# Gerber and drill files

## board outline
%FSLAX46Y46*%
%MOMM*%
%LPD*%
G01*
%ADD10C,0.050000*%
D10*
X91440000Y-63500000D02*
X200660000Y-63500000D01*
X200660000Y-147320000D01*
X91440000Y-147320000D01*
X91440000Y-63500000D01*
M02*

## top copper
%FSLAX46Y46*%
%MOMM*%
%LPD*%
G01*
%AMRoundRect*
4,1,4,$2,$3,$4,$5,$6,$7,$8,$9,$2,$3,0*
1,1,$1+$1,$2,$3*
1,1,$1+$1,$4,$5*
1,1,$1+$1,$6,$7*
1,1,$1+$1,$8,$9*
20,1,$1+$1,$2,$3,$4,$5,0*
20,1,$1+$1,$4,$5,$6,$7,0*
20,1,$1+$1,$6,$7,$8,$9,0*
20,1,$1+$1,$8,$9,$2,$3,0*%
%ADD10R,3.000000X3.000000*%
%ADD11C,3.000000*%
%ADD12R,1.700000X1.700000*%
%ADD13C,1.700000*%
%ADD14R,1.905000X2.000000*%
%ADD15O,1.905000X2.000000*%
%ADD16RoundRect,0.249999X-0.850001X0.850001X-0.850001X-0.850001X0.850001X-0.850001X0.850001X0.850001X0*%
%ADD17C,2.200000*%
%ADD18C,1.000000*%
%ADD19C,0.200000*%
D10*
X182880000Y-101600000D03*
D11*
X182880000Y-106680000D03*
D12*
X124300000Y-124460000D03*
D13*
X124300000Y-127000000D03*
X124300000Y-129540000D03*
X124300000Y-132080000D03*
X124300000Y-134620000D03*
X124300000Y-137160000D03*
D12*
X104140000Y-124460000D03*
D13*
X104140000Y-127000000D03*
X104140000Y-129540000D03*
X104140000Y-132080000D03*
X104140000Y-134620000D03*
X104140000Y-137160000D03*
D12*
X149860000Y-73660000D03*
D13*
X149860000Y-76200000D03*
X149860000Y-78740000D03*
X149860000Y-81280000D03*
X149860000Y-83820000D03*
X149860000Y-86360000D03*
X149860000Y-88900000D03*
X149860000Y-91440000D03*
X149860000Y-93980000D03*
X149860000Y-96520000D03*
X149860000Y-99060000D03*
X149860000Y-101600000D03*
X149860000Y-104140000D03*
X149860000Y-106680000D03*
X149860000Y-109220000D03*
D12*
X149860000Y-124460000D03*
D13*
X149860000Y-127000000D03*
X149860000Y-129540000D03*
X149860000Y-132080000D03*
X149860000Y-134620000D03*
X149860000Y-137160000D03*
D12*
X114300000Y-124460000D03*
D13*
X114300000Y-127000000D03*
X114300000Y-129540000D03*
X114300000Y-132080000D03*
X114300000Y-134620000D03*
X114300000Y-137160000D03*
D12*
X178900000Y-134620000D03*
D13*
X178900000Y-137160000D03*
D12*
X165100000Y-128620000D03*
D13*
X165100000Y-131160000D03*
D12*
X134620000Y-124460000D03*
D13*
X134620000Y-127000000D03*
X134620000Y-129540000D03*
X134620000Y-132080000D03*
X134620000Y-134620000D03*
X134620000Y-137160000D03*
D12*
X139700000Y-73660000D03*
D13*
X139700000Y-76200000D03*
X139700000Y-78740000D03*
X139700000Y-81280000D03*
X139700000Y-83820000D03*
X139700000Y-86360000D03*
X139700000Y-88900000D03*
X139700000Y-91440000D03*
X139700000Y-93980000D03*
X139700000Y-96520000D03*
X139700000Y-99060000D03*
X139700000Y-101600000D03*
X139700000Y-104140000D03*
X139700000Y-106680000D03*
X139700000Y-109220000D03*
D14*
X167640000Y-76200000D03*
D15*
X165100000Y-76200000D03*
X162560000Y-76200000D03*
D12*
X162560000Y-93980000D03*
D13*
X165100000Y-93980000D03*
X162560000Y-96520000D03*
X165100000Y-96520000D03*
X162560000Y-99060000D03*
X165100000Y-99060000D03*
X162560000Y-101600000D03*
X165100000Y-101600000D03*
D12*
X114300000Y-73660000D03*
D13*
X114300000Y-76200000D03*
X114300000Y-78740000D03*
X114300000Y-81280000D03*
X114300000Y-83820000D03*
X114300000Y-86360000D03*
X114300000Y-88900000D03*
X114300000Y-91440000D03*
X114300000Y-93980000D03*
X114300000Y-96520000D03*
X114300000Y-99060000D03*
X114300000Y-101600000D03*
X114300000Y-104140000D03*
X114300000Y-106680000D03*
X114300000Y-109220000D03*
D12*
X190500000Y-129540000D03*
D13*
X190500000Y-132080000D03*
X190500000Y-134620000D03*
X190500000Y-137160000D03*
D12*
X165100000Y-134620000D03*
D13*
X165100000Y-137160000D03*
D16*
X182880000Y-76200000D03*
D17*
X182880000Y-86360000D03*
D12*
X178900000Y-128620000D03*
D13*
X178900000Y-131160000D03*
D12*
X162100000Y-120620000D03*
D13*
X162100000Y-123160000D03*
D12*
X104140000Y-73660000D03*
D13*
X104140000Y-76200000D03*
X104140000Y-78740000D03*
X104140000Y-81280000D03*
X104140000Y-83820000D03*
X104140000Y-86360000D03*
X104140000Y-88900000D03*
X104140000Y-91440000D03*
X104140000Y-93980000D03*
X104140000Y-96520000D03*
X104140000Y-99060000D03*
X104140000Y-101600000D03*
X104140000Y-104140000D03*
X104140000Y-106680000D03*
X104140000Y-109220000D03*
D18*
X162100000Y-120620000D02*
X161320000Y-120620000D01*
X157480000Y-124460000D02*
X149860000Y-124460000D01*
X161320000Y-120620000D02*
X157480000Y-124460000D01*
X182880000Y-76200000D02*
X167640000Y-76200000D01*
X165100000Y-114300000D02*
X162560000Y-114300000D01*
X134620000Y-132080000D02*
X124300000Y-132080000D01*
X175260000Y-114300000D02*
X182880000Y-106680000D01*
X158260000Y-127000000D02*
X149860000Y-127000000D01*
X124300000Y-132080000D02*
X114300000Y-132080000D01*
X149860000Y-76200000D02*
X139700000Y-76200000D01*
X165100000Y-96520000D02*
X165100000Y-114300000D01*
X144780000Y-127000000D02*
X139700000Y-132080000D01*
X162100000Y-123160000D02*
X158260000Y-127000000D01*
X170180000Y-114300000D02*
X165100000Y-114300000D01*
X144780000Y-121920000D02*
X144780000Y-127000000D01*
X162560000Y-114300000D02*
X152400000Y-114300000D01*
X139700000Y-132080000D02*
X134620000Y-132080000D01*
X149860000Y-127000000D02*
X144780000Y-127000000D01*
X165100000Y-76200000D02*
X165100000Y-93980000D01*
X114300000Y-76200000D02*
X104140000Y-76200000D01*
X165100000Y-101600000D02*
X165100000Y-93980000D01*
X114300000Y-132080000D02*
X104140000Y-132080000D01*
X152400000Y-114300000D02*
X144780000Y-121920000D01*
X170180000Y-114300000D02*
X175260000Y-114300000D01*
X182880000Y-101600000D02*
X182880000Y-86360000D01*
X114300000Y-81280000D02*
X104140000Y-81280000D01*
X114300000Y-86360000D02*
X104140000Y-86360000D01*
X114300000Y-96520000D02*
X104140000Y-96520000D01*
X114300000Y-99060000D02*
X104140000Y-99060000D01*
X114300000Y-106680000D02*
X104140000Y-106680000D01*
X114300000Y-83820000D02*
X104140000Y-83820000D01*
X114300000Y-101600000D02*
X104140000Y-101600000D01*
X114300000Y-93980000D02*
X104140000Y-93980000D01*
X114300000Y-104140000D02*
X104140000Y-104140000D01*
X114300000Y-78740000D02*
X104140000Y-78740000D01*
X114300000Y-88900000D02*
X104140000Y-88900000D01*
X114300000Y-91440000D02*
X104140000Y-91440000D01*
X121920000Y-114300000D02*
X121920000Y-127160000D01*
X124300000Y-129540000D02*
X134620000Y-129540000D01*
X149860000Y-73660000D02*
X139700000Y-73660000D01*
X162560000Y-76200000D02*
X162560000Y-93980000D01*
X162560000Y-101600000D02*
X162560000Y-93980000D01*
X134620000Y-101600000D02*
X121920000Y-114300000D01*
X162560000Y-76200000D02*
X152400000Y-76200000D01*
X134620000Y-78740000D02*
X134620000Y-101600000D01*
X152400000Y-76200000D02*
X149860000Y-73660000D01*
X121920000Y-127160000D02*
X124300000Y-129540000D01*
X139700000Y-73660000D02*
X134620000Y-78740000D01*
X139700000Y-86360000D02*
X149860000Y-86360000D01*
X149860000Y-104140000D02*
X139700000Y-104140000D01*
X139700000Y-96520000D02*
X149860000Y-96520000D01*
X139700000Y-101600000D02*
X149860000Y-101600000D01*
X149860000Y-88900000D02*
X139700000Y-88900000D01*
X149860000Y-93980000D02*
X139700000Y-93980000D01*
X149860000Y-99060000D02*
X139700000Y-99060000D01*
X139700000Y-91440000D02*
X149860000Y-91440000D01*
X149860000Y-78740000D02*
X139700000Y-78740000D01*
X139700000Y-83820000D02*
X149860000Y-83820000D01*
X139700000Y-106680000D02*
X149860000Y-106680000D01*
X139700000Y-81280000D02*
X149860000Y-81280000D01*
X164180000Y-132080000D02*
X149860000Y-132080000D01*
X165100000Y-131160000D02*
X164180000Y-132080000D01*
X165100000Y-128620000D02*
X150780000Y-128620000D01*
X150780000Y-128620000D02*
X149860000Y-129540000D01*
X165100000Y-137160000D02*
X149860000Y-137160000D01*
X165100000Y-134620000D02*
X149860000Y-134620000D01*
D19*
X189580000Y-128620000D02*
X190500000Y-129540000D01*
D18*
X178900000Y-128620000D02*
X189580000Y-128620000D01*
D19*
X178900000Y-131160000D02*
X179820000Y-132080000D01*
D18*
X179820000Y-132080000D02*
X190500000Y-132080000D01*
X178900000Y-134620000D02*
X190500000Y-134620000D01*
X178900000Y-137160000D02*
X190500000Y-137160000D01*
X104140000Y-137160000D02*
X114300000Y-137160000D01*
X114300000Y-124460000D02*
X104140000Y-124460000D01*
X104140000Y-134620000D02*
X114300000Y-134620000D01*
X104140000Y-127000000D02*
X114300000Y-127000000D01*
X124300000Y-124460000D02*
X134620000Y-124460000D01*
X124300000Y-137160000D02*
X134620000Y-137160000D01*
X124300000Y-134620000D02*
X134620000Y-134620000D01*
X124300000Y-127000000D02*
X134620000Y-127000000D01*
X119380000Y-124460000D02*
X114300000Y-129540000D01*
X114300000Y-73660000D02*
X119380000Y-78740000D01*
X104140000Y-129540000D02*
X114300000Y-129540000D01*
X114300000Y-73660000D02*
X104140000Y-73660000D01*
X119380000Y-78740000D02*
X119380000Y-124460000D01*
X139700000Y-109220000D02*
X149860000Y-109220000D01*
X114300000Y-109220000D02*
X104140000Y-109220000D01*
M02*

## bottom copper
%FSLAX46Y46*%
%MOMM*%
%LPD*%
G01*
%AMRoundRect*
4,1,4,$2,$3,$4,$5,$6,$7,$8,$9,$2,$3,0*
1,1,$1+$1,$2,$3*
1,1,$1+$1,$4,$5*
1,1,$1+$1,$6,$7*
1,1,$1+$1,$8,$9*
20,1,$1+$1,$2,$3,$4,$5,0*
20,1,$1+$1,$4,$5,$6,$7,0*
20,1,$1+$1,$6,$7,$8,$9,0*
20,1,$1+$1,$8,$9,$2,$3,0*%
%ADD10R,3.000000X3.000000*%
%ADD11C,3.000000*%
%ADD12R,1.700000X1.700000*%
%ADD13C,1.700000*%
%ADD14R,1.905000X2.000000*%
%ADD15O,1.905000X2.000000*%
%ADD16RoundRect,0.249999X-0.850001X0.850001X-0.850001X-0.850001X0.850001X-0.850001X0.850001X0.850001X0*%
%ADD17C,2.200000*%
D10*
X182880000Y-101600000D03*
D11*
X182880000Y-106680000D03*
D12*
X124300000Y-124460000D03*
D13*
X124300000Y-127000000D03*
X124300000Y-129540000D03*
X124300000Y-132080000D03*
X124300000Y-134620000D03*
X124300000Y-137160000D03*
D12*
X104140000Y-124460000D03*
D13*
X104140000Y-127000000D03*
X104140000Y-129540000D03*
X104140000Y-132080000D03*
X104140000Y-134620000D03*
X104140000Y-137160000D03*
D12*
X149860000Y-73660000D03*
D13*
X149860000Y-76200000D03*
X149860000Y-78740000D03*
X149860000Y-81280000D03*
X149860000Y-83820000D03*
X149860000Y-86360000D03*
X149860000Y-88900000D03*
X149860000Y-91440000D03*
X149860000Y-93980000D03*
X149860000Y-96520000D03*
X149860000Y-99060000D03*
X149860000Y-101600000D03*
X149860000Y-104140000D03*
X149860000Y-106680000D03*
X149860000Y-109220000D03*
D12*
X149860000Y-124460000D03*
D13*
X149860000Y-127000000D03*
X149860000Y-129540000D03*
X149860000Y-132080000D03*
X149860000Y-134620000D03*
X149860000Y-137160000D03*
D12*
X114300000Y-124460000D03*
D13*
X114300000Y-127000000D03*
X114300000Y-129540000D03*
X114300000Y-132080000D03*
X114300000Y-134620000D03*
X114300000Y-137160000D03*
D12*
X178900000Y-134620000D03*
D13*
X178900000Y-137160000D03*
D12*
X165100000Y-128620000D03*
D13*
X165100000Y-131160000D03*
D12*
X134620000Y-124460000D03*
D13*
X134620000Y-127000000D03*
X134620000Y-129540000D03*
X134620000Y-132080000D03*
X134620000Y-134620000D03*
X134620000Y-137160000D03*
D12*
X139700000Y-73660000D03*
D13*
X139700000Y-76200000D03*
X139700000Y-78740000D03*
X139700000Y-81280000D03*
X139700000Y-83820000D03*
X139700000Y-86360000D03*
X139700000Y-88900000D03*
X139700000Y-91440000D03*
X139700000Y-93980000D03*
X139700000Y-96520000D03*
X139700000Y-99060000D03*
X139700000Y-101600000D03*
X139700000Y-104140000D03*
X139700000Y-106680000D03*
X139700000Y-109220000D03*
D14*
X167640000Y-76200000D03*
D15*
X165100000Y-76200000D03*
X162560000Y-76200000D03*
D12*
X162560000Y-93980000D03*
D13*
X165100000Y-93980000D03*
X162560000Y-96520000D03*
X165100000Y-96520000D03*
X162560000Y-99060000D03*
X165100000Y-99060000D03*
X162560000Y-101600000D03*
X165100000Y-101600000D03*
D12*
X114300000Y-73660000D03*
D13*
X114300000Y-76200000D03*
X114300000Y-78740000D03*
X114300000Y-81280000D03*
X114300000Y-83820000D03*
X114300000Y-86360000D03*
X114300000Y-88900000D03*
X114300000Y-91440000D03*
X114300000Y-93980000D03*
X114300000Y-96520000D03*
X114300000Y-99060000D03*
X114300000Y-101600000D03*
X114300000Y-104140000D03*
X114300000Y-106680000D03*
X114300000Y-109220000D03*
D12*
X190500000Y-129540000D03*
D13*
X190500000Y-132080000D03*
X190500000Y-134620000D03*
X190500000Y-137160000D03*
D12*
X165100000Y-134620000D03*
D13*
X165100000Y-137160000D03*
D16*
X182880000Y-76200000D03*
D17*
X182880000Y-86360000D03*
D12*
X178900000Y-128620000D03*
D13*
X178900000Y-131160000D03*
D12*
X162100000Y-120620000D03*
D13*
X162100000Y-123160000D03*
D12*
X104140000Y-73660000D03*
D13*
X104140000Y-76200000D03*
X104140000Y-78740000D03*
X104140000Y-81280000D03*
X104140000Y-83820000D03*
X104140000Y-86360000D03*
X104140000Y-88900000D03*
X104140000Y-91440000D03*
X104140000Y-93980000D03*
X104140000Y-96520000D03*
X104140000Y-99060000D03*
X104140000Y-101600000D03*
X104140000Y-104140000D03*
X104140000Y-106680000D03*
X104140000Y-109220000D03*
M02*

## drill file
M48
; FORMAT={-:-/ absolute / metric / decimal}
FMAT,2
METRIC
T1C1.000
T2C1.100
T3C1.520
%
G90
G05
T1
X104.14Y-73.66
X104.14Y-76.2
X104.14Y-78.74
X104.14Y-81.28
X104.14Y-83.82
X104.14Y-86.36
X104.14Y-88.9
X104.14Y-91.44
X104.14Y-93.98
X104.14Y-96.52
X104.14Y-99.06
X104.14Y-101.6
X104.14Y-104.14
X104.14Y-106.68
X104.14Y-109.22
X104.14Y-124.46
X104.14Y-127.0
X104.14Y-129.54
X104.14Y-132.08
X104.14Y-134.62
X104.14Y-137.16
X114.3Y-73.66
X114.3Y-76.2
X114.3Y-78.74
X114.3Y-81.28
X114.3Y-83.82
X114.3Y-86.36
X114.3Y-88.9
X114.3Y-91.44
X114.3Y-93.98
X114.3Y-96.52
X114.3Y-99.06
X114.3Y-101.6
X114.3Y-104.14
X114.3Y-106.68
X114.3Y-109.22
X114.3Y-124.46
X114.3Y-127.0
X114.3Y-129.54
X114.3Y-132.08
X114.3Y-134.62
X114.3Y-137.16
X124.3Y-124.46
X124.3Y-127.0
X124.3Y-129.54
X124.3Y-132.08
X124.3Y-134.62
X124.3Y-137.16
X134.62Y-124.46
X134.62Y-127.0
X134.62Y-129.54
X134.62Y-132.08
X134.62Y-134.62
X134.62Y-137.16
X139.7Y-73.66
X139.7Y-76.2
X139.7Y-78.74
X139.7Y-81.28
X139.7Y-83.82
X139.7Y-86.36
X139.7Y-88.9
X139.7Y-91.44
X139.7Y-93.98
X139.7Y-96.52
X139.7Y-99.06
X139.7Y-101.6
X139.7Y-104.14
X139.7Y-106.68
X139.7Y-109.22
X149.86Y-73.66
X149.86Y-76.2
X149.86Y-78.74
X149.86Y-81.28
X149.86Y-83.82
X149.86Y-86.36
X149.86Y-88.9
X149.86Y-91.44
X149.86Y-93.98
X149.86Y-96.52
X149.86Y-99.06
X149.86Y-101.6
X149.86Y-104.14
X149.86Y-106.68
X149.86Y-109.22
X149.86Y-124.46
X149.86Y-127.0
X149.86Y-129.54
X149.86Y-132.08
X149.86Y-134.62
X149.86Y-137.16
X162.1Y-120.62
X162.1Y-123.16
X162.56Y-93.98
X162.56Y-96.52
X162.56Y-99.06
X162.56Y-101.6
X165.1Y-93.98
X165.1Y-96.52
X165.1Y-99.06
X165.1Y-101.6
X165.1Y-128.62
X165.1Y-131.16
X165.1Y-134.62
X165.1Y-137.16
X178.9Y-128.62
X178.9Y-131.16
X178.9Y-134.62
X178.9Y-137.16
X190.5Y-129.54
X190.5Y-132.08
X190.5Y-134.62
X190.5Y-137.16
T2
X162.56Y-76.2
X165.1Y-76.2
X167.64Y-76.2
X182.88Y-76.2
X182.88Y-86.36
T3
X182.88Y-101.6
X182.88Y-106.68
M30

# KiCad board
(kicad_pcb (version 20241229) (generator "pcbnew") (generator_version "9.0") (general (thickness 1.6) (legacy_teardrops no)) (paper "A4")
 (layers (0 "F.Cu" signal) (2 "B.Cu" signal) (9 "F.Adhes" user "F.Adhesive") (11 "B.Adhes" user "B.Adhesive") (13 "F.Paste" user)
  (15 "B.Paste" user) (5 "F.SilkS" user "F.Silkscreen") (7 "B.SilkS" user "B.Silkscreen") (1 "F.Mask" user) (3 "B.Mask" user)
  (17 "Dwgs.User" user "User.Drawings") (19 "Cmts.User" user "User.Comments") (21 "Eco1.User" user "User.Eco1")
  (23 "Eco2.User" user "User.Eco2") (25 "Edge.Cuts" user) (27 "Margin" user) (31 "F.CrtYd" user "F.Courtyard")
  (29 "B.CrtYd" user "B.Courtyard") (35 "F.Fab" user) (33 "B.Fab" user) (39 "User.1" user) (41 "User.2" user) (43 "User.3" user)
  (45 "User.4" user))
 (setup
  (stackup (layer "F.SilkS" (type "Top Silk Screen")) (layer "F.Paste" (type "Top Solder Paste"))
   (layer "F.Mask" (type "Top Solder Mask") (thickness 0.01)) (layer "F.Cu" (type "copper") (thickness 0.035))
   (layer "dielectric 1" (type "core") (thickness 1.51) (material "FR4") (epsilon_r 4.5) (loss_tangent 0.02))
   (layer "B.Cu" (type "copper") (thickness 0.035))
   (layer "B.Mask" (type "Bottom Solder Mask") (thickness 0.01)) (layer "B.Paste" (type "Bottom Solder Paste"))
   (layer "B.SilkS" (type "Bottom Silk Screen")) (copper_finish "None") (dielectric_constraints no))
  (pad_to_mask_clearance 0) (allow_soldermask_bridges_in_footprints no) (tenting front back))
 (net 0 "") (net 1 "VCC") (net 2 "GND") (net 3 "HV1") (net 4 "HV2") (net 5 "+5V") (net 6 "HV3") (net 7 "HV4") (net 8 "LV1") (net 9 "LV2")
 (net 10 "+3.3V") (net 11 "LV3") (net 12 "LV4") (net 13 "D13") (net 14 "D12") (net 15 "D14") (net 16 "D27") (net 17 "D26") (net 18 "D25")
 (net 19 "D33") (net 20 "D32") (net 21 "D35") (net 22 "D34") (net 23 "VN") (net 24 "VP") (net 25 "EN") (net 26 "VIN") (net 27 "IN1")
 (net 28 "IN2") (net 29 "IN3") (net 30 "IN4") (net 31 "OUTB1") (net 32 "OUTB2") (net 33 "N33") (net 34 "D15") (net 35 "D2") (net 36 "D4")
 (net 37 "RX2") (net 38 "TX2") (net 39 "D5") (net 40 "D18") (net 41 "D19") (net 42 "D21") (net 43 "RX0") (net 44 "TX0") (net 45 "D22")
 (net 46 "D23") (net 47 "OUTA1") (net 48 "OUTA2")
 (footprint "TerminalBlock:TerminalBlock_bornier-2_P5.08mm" (layer "F.Cu") (at 182.88 101.6 -90)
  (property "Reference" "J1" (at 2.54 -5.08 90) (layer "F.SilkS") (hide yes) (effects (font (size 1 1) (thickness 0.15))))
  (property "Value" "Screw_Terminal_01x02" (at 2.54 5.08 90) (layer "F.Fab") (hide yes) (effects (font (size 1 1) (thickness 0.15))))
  (pad "1" thru_hole rect (at 0 0 270) (size 3 3) (drill 1.52) (layers "*.Cu" "*.Mask") (remove_unused_layers no) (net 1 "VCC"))
  (pad "2" thru_hole circle (at 5.08 0 270) (size 3 3) (drill 1.52) (layers "*.Cu" "*.Mask") (remove_unused_layers no) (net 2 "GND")))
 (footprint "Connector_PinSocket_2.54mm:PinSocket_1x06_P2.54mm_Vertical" (layer "F.Cu") (at 124.3 124.46)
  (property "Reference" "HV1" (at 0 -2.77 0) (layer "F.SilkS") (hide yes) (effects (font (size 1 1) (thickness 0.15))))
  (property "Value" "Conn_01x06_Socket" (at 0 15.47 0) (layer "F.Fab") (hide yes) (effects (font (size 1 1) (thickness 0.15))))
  (pad "1" thru_hole rect (at 0 0) (size 1.7 1.7) (drill 1) (layers "*.Cu" "*.Mask") (remove_unused_layers no) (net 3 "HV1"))
  (pad "2" thru_hole circle (at 0 2.54) (size 1.7 1.7) (drill 1) (layers "*.Cu" "*.Mask") (remove_unused_layers no) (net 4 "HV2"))
  (pad "3" thru_hole circle (at 0 5.08) (size 1.7 1.7) (drill 1) (layers "*.Cu" "*.Mask") (remove_unused_layers no) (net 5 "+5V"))
  (pad "4" thru_hole circle (at 0 7.62) (size 1.7 1.7) (drill 1) (layers "*.Cu" "*.Mask") (remove_unused_layers no) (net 2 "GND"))
  (pad "5" thru_hole circle (at 0 10.16) (size 1.7 1.7) (drill 1) (layers "*.Cu" "*.Mask") (remove_unused_layers no) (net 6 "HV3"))
  (pad "6" thru_hole circle (at 0 12.7) (size 1.7 1.7) (drill 1) (layers "*.Cu" "*.Mask") (remove_unused_layers no) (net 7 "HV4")))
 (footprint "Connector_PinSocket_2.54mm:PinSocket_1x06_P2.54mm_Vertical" (layer "F.Cu") (at 104.14 124.46)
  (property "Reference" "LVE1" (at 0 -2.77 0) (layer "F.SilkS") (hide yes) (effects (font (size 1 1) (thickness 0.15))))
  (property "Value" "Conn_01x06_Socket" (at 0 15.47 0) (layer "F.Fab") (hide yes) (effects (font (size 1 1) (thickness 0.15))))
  (pad "1" thru_hole rect (at 0 0) (size 1.7 1.7) (drill 1) (layers "*.Cu" "*.Mask") (remove_unused_layers no) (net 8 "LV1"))
  (pad "2" thru_hole circle (at 0 2.54) (size 1.7 1.7) (drill 1) (layers "*.Cu" "*.Mask") (remove_unused_layers no) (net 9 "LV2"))
  (pad "3" thru_hole circle (at 0 5.08) (size 1.7 1.7) (drill 1) (layers "*.Cu" "*.Mask") (remove_unused_layers no) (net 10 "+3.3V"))
  (pad "4" thru_hole circle (at 0 7.62) (size 1.7 1.7) (drill 1) (layers "*.Cu" "*.Mask") (remove_unused_layers no) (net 2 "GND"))
  (pad "5" thru_hole circle (at 0 10.16) (size 1.7 1.7) (drill 1) (layers "*.Cu" "*.Mask") (remove_unused_layers no) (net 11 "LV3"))
  (pad "6" thru_hole circle (at 0 12.7) (size 1.7 1.7) (drill 1) (layers "*.Cu" "*.Mask") (remove_unused_layers no) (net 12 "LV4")))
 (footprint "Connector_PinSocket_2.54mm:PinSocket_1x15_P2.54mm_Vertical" (layer "F.Cu") (at 149.86 73.66)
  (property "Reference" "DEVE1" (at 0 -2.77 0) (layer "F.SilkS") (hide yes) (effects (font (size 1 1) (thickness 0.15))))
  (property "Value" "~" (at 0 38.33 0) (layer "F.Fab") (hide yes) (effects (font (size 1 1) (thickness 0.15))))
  (pad "1" thru_hole rect (at 0 0) (size 1.7 1.7) (drill 1) (layers "*.Cu" "*.Mask") (remove_unused_layers no) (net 5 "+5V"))
  (pad "2" thru_hole circle (at 0 2.54) (size 1.7 1.7) (drill 1) (layers "*.Cu" "*.Mask") (remove_unused_layers no) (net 2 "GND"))
  (pad "3" thru_hole circle (at 0 5.08) (size 1.7 1.7) (drill 1) (layers "*.Cu" "*.Mask") (remove_unused_layers no) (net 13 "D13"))
  (pad "4" thru_hole circle (at 0 7.62) (size 1.7 1.7) (drill 1) (layers "*.Cu" "*.Mask") (remove_unused_layers no) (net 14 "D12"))
  (pad "5" thru_hole circle (at 0 10.16) (size 1.7 1.7) (drill 1) (layers "*.Cu" "*.Mask") (remove_unused_layers no) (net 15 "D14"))
  (pad "6" thru_hole circle (at 0 12.7) (size 1.7 1.7) (drill 1) (layers "*.Cu" "*.Mask") (remove_unused_layers no) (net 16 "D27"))
  (pad "7" thru_hole circle (at 0 15.24) (size 1.7 1.7) (drill 1) (layers "*.Cu" "*.Mask") (remove_unused_layers no) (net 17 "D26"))
  (pad "8" thru_hole circle (at 0 17.78) (size 1.7 1.7) (drill 1) (layers "*.Cu" "*.Mask") (remove_unused_layers no) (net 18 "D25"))
  (pad "9" thru_hole circle (at 0 20.32) (size 1.7 1.7) (drill 1) (layers "*.Cu" "*.Mask") (remove_unused_layers no) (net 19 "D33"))
  (pad "10" thru_hole circle (at 0 22.86) (size 1.7 1.7) (drill 1) (layers "*.Cu" "*.Mask") (remove_unused_layers no) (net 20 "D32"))
  (pad "11" thru_hole circle (at 0 25.4) (size 1.7 1.7) (drill 1) (layers "*.Cu" "*.Mask") (remove_unused_layers no) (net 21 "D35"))
  (pad "12" thru_hole circle (at 0 27.94) (size 1.7 1.7) (drill 1) (layers "*.Cu" "*.Mask") (remove_unused_layers no) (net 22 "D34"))
  (pad "13" thru_hole circle (at 0 30.48) (size 1.7 1.7) (drill 1) (layers "*.Cu" "*.Mask") (remove_unused_layers no) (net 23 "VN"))
  (pad "14" thru_hole circle (at 0 33.02) (size 1.7 1.7) (drill 1) (layers "*.Cu" "*.Mask") (remove_unused_layers no) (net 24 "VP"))
  (pad "15" thru_hole circle (at 0 35.56) (size 1.7 1.7) (drill 1) (layers "*.Cu" "*.Mask") (remove_unused_layers no) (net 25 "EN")))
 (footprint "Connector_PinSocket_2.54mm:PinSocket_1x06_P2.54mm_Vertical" (layer "F.Cu") (at 149.86 124.46)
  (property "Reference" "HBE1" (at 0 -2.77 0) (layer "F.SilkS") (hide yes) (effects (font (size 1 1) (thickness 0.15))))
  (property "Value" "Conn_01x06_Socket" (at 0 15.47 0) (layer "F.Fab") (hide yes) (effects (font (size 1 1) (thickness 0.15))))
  (pad "1" thru_hole rect (at 0 0) (size 1.7 1.7) (drill 1) (layers "*.Cu" "*.Mask") (remove_unused_layers no) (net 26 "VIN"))
  (pad "2" thru_hole circle (at 0 2.54) (size 1.7 1.7) (drill 1) (layers "*.Cu" "*.Mask") (remove_unused_layers no) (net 2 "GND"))
  (pad "3" thru_hole circle (at 0 5.08) (size 1.7 1.7) (drill 1) (layers "*.Cu" "*.Mask") (remove_unused_layers no) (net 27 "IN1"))
  (pad "4" thru_hole circle (at 0 7.62) (size 1.7 1.7) (drill 1) (layers "*.Cu" "*.Mask") (remove_unused_layers no) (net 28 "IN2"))
  (pad "5" thru_hole circle (at 0 10.16) (size 1.7 1.7) (drill 1) (layers "*.Cu" "*.Mask") (remove_unused_layers no) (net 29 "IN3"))
  (pad "6" thru_hole circle (at 0 12.7) (size 1.7 1.7) (drill 1) (layers "*.Cu" "*.Mask") (remove_unused_layers no) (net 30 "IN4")))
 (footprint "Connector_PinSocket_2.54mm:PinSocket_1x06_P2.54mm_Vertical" (layer "F.Cu") (at 114.3 124.46)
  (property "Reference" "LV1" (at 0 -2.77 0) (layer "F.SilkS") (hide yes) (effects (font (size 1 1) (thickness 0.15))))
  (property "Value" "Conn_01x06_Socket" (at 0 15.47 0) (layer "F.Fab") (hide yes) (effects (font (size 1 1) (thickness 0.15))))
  (pad "1" thru_hole rect (at 0 0) (size 1.7 1.7) (drill 1) (layers "*.Cu" "*.Mask") (remove_unused_layers no) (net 8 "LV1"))
  (pad "2" thru_hole circle (at 0 2.54) (size 1.7 1.7) (drill 1) (layers "*.Cu" "*.Mask") (remove_unused_layers no) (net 9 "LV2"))
  (pad "3" thru_hole circle (at 0 5.08) (size 1.7 1.7) (drill 1) (layers "*.Cu" "*.Mask") (remove_unused_layers no) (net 10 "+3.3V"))
  (pad "4" thru_hole circle (at 0 7.62) (size 1.7 1.7) (drill 1) (layers "*.Cu" "*.Mask") (remove_unused_layers no) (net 2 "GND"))
  (pad "5" thru_hole circle (at 0 10.16) (size 1.7 1.7) (drill 1) (layers "*.Cu" "*.Mask") (remove_unused_layers no) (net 11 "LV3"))
  (pad "6" thru_hole circle (at 0 12.7) (size 1.7 1.7) (drill 1) (layers "*.Cu" "*.Mask") (remove_unused_layers no) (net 12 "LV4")))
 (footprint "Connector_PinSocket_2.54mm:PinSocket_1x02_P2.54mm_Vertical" (layer "F.Cu") (at 178.9 134.62)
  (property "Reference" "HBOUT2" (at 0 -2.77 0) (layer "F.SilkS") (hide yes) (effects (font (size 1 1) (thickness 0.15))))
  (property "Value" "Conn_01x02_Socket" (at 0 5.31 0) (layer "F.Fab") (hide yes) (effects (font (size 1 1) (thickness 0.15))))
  (pad "1" thru_hole rect (at 0 0) (size 1.7 1.7) (drill 1) (layers "*.Cu" "*.Mask") (remove_unused_layers no) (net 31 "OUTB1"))
  (pad "2" thru_hole circle (at 0 2.54) (size 1.7 1.7) (drill 1) (layers "*.Cu" "*.Mask") (remove_unused_layers no) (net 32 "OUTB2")))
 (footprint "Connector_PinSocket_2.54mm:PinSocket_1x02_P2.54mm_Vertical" (layer "F.Cu") (at 165.1 128.62)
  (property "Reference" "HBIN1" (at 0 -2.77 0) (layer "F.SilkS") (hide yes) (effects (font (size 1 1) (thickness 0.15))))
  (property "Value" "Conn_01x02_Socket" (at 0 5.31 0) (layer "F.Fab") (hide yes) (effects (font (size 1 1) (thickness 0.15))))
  (pad "1" thru_hole rect (at 0 0) (size 1.7 1.7) (drill 1) (layers "*.Cu" "*.Mask") (remove_unused_layers no) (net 27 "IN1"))
  (pad "2" thru_hole circle (at 0 2.54) (size 1.7 1.7) (drill 1) (layers "*.Cu" "*.Mask") (remove_unused_layers no) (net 28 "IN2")))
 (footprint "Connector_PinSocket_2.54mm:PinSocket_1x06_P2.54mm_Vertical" (layer "F.Cu") (at 134.62 124.46)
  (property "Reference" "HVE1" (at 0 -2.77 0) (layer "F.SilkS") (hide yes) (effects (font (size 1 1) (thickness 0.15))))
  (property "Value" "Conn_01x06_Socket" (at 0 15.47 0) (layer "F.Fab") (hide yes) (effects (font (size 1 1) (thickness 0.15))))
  (pad "1" thru_hole rect (at 0 0) (size 1.7 1.7) (drill 1) (layers "*.Cu" "*.Mask") (remove_unused_layers no) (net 3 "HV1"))
  (pad "2" thru_hole circle (at 0 2.54) (size 1.7 1.7) (drill 1) (layers "*.Cu" "*.Mask") (remove_unused_layers no) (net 4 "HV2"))
  (pad "3" thru_hole circle (at 0 5.08) (size 1.7 1.7) (drill 1) (layers "*.Cu" "*.Mask") (remove_unused_layers no) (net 5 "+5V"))
  (pad "4" thru_hole circle (at 0 7.62) (size 1.7 1.7) (drill 1) (layers "*.Cu" "*.Mask") (remove_unused_layers no) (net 2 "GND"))
  (pad "5" thru_hole circle (at 0 10.16) (size 1.7 1.7) (drill 1) (layers "*.Cu" "*.Mask") (remove_unused_layers no) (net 6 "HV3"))
  (pad "6" thru_hole circle (at 0 12.7) (size 1.7 1.7) (drill 1) (layers "*.Cu" "*.Mask") (remove_unused_layers no) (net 7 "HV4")))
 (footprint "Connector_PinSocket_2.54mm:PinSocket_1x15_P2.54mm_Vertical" (layer "F.Cu") (at 139.7 73.66)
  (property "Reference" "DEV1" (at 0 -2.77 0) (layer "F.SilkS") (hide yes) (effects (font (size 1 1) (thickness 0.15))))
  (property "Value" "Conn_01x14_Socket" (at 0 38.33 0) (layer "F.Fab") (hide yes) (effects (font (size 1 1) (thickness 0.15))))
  (pad "1" thru_hole rect (at 0 0) (size 1.7 1.7) (drill 1) (layers "*.Cu" "*.Mask") (remove_unused_layers no) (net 5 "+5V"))
  (pad "2" thru_hole circle (at 0 2.54) (size 1.7 1.7) (drill 1) (layers "*.Cu" "*.Mask") (remove_unused_layers no) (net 2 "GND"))
  (pad "3" thru_hole circle (at 0 5.08) (size 1.7 1.7) (drill 1) (layers "*.Cu" "*.Mask") (remove_unused_layers no) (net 13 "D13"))
  (pad "4" thru_hole circle (at 0 7.62) (size 1.7 1.7) (drill 1) (layers "*.Cu" "*.Mask") (remove_unused_layers no) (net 14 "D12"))
  (pad "5" thru_hole circle (at 0 10.16) (size 1.7 1.7) (drill 1) (layers "*.Cu" "*.Mask") (remove_unused_layers no) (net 15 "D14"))
  (pad "6" thru_hole circle (at 0 12.7) (size 1.7 1.7) (drill 1) (layers "*.Cu" "*.Mask") (remove_unused_layers no) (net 16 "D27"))
  (pad "7" thru_hole circle (at 0 15.24) (size 1.7 1.7) (drill 1) (layers "*.Cu" "*.Mask") (remove_unused_layers no) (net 17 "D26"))
  (pad "8" thru_hole circle (at 0 17.78) (size 1.7 1.7) (drill 1) (layers "*.Cu" "*.Mask") (remove_unused_layers no) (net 18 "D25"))
  (pad "9" thru_hole circle (at 0 20.32) (size 1.7 1.7) (drill 1) (layers "*.Cu" "*.Mask") (remove_unused_layers no) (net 19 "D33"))
  (pad "10" thru_hole circle (at 0 22.86) (size 1.7 1.7) (drill 1) (layers "*.Cu" "*.Mask") (remove_unused_layers no) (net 20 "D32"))
  (pad "11" thru_hole circle (at 0 25.4) (size 1.7 1.7) (drill 1) (layers "*.Cu" "*.Mask") (remove_unused_layers no) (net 21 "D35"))
  (pad "12" thru_hole circle (at 0 27.94) (size 1.7 1.7) (drill 1) (layers "*.Cu" "*.Mask") (remove_unused_layers no) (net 22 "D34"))
  (pad "13" thru_hole circle (at 0 30.48) (size 1.7 1.7) (drill 1) (layers "*.Cu" "*.Mask") (remove_unused_layers no) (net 23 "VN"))
  (pad "14" thru_hole circle (at 0 33.02) (size 1.7 1.7) (drill 1) (layers "*.Cu" "*.Mask") (remove_unused_layers no) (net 24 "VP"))
  (pad "15" thru_hole circle (at 0 35.56) (size 1.7 1.7) (drill 1) (layers "*.Cu" "*.Mask") (remove_unused_layers no) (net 25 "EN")))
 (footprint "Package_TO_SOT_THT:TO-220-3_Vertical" (layer "F.Cu") (at 167.64 76.2 180)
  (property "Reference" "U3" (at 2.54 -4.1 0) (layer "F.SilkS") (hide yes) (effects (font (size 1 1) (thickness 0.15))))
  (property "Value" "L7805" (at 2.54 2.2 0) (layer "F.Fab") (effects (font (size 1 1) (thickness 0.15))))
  (pad "1" thru_hole rect (at 0 0 180) (size 1.905 2) (drill 1.1) (layers "*.Cu" "*.Mask") (remove_unused_layers no) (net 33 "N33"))
  (pad "2" thru_hole oval (at 2.54 0 180) (size 1.905 2) (drill 1.1) (layers "*.Cu" "*.Mask") (remove_unused_layers no) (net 2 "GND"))
  (pad "3" thru_hole oval (at 5.08 0 180) (size 1.905 2) (drill 1.1) (layers "*.Cu" "*.Mask") (remove_unused_layers no) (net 5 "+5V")))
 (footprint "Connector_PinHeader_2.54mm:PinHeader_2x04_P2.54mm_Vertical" (layer "F.Cu") (at 162.56 93.98)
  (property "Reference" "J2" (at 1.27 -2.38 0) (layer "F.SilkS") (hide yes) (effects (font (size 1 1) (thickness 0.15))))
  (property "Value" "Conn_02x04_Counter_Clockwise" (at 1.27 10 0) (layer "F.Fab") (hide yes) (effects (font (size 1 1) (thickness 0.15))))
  (pad "1" thru_hole rect (at 0 0) (size 1.7 1.7) (drill 1) (layers "*.Cu" "*.Mask") (remove_unused_layers no) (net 5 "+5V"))
  (pad "2" thru_hole circle (at 2.54 0) (size 1.7 1.7) (drill 1) (layers "*.Cu" "*.Mask") (remove_unused_layers no) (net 2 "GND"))
  (pad "3" thru_hole circle (at 0 2.54) (size 1.7 1.7) (drill 1) (layers "*.Cu" "*.Mask") (remove_unused_layers no) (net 5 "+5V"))
  (pad "4" thru_hole circle (at 2.54 2.54) (size 1.7 1.7) (drill 1) (layers "*.Cu" "*.Mask") (remove_unused_layers no) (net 2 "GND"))
  (pad "5" thru_hole circle (at 0 5.08) (size 1.7 1.7) (drill 1) (layers "*.Cu" "*.Mask") (remove_unused_layers no) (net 5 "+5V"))
  (pad "6" thru_hole circle (at 2.54 5.08) (size 1.7 1.7) (drill 1) (layers "*.Cu" "*.Mask") (remove_unused_layers no) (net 2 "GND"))
  (pad "7" thru_hole circle (at 0 7.62) (size 1.7 1.7) (drill 1) (layers "*.Cu" "*.Mask") (remove_unused_layers no) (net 5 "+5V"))
  (pad "8" thru_hole circle (at 2.54 7.62) (size 1.7 1.7) (drill 1) (layers "*.Cu" "*.Mask") (remove_unused_layers no) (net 2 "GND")))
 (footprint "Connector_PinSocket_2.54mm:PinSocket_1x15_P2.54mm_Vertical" (layer "F.Cu") (at 114.3 73.66)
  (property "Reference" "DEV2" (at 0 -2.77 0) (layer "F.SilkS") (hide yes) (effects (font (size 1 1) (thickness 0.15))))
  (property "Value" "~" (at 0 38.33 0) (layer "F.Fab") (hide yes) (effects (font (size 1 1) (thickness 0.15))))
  (pad "1" thru_hole rect (at 0 0) (size 1.7 1.7) (drill 1) (layers "*.Cu" "*.Mask") (remove_unused_layers no) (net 10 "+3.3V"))
  (pad "2" thru_hole circle (at 0 2.54) (size 1.7 1.7) (drill 1) (layers "*.Cu" "*.Mask") (remove_unused_layers no) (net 2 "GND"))
  (pad "3" thru_hole circle (at 0 5.08) (size 1.7 1.7) (drill 1) (layers "*.Cu" "*.Mask") (remove_unused_layers no) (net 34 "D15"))
  (pad "4" thru_hole circle (at 0 7.62) (size 1.7 1.7) (drill 1) (layers "*.Cu" "*.Mask") (remove_unused_layers no) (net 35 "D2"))
  (pad "5" thru_hole circle (at 0 10.16) (size 1.7 1.7) (drill 1) (layers "*.Cu" "*.Mask") (remove_unused_layers no) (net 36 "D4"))
  (pad "6" thru_hole circle (at 0 12.7) (size 1.7 1.7) (drill 1) (layers "*.Cu" "*.Mask") (remove_unused_layers no) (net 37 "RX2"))
  (pad "7" thru_hole circle (at 0 15.24) (size 1.7 1.7) (drill 1) (layers "*.Cu" "*.Mask") (remove_unused_layers no) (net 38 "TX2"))
  (pad "8" thru_hole circle (at 0 17.78) (size 1.7 1.7) (drill 1) (layers "*.Cu" "*.Mask") (remove_unused_layers no) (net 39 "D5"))
  (pad "9" thru_hole circle (at 0 20.32) (size 1.7 1.7) (drill 1) (layers "*.Cu" "*.Mask") (remove_unused_layers no) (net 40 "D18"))
  (pad "10" thru_hole circle (at 0 22.86) (size 1.7 1.7) (drill 1) (layers "*.Cu" "*.Mask") (remove_unused_layers no) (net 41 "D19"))
  (pad "11" thru_hole circle (at 0 25.4) (size 1.7 1.7) (drill 1) (layers "*.Cu" "*.Mask") (remove_unused_layers no) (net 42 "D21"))
  (pad "12" thru_hole circle (at 0 27.94) (size 1.7 1.7) (drill 1) (layers "*.Cu" "*.Mask") (remove_unused_layers no) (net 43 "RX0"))
  (pad "13" thru_hole circle (at 0 30.48) (size 1.7 1.7) (drill 1) (layers "*.Cu" "*.Mask") (remove_unused_layers no) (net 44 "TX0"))
  (pad "14" thru_hole circle (at 0 33.02) (size 1.7 1.7) (drill 1) (layers "*.Cu" "*.Mask") (remove_unused_layers no) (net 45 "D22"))
  (pad "15" thru_hole circle (at 0 35.56) (size 1.7 1.7) (drill 1) (layers "*.Cu" "*.Mask") (remove_unused_layers no) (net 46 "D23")))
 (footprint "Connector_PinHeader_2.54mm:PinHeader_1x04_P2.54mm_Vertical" (layer "F.Cu") (at 190.5 129.54)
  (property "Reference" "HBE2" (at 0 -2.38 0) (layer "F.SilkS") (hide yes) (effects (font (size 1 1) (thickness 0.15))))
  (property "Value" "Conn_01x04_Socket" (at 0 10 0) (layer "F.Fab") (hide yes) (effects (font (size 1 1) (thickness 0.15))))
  (pad "1" thru_hole rect (at 0 0) (size 1.7 1.7) (drill 1) (layers "*.Cu" "*.Mask") (remove_unused_layers no) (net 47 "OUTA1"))
  (pad "2" thru_hole circle (at 0 2.54) (size 1.7 1.7) (drill 1) (layers "*.Cu" "*.Mask") (remove_unused_layers no) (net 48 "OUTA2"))
  (pad "3" thru_hole circle (at 0 5.08) (size 1.7 1.7) (drill 1) (layers "*.Cu" "*.Mask") (remove_unused_layers no) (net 31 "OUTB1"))
  (pad "4" thru_hole circle (at 0 7.62) (size 1.7 1.7) (drill 1) (layers "*.Cu" "*.Mask") (remove_unused_layers no) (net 32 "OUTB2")))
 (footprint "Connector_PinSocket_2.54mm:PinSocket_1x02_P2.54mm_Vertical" (layer "F.Cu") (at 165.1 134.62)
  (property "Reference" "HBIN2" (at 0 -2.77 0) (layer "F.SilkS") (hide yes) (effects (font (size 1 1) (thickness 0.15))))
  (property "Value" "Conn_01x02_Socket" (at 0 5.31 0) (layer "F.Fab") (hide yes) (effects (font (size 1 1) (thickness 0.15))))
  (pad "1" thru_hole rect (at 0 0) (size 1.7 1.7) (drill 1) (layers "*.Cu" "*.Mask") (remove_unused_layers no) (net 29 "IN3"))
  (pad "2" thru_hole circle (at 0 2.54) (size 1.7 1.7) (drill 1) (layers "*.Cu" "*.Mask") (remove_unused_layers no) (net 30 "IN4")))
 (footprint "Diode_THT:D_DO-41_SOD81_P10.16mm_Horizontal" (layer "F.Cu") (at 182.88 76.2 -90)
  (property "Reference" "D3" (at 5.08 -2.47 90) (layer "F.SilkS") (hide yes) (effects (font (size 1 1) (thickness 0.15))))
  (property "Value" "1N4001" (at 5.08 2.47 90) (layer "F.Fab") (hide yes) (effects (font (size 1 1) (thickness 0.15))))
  (pad "1" thru_hole roundrect (at 0 0 270) (size 2.2 2.2) (drill 1.1) (layers "*.Cu" "*.Mask") (remove_unused_layers no)
   (roundrect_rratio 0.113636) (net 33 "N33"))
  (pad "2" thru_hole circle (at 10.16 0 270) (size 2.2 2.2) (drill 1.1) (layers "*.Cu" "*.Mask") (remove_unused_layers no) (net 1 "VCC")))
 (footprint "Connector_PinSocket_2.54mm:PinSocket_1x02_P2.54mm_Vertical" (layer "F.Cu") (at 178.9 128.62)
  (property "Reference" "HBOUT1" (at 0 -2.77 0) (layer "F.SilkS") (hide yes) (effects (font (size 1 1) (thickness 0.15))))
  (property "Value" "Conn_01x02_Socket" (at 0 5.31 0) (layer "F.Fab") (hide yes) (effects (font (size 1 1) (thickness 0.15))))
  (pad "1" thru_hole rect (at 0 0) (size 1.7 1.7) (drill 1) (layers "*.Cu" "*.Mask") (remove_unused_layers no) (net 47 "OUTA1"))
  (pad "2" thru_hole circle (at 0 2.54) (size 1.7 1.7) (drill 1) (layers "*.Cu" "*.Mask") (remove_unused_layers no) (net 48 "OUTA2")))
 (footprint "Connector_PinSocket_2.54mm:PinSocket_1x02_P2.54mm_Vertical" (layer "F.Cu") (at 162.1 120.62)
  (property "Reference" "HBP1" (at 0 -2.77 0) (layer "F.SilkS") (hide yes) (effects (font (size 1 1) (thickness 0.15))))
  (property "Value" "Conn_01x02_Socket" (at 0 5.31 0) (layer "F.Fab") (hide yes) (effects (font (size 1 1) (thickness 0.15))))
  (pad "1" thru_hole rect (at 0 0) (size 1.7 1.7) (drill 1) (layers "*.Cu" "*.Mask") (remove_unused_layers no) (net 26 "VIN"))
  (pad "2" thru_hole circle (at 0 2.54) (size 1.7 1.7) (drill 1) (layers "*.Cu" "*.Mask") (remove_unused_layers no) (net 2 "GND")))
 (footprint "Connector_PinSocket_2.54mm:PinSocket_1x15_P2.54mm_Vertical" (layer "F.Cu") (at 104.14 73.66)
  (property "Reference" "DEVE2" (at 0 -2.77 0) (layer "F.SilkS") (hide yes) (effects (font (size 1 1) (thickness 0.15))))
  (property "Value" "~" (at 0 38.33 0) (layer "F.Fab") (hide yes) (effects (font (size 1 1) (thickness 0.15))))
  (pad "1" thru_hole rect (at 0 0) (size 1.7 1.7) (drill 1) (layers "*.Cu" "*.Mask") (remove_unused_layers no) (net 10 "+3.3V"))
  (pad "2" thru_hole circle (at 0 2.54) (size 1.7 1.7) (drill 1) (layers "*.Cu" "*.Mask") (remove_unused_layers no) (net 2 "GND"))
  (pad "3" thru_hole circle (at 0 5.08) (size 1.7 1.7) (drill 1) (layers "*.Cu" "*.Mask") (remove_unused_layers no) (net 34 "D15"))
  (pad "4" thru_hole circle (at 0 7.62) (size 1.7 1.7) (drill 1) (layers "*.Cu" "*.Mask") (remove_unused_layers no) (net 35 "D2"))
  (pad "5" thru_hole circle (at 0 10.16) (size 1.7 1.7) (drill 1) (layers "*.Cu" "*.Mask") (remove_unused_layers no) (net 36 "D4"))
  (pad "6" thru_hole circle (at 0 12.7) (size 1.7 1.7) (drill 1) (layers "*.Cu" "*.Mask") (remove_unused_layers no) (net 37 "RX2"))
  (pad "7" thru_hole circle (at 0 15.24) (size 1.7 1.7) (drill 1) (layers "*.Cu" "*.Mask") (remove_unused_layers no) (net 38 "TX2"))
  (pad "8" thru_hole circle (at 0 17.78) (size 1.7 1.7) (drill 1) (layers "*.Cu" "*.Mask") (remove_unused_layers no) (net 39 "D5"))
  (pad "9" thru_hole circle (at 0 20.32) (size 1.7 1.7) (drill 1) (layers "*.Cu" "*.Mask") (remove_unused_layers no) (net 40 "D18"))
  (pad "10" thru_hole circle (at 0 22.86) (size 1.7 1.7) (drill 1) (layers "*.Cu" "*.Mask") (remove_unused_layers no) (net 41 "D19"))
  (pad "11" thru_hole circle (at 0 25.4) (size 1.7 1.7) (drill 1) (layers "*.Cu" "*.Mask") (remove_unused_layers no) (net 42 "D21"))
  (pad "12" thru_hole circle (at 0 27.94) (size 1.7 1.7) (drill 1) (layers "*.Cu" "*.Mask") (remove_unused_layers no) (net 43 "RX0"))
  (pad "13" thru_hole circle (at 0 30.48) (size 1.7 1.7) (drill 1) (layers "*.Cu" "*.Mask") (remove_unused_layers no) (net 44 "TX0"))
  (pad "14" thru_hole circle (at 0 33.02) (size 1.7 1.7) (drill 1) (layers "*.Cu" "*.Mask") (remove_unused_layers no) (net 45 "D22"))
  (pad "15" thru_hole circle (at 0 35.56) (size 1.7 1.7) (drill 1) (layers "*.Cu" "*.Mask") (remove_unused_layers no) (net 46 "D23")))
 (gr_rect (start 91.44 63.5) (end 200.66 147.32) (stroke (width 0.05) (type solid)) (fill no) (layer "Edge.Cuts"))
 (segment (start 162.1 120.62) (end 161.32 120.62) (width 1) (layer "F.Cu") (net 26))
 (segment (start 157.48 124.46) (end 149.86 124.46) (width 1) (layer "F.Cu") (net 26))
 (segment (start 161.32 120.62) (end 157.48 124.46) (width 1) (layer "F.Cu") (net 26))
 (segment (start 182.88 76.2) (end 167.64 76.2) (width 1) (layer "F.Cu") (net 33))
 (segment (start 165.1 114.3) (end 162.56 114.3) (width 1) (layer "F.Cu") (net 2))
 (segment (start 134.62 132.08) (end 124.3 132.08) (width 1) (layer "F.Cu") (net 2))
 (segment (start 175.26 114.3) (end 182.88 106.68) (width 1) (layer "F.Cu") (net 2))
 (segment (start 158.26 127) (end 149.86 127) (width 1) (layer "F.Cu") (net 2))
 (segment (start 124.3 132.08) (end 114.3 132.08) (width 1) (layer "F.Cu") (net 2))
 (segment (start 149.86 76.2) (end 139.7 76.2) (width 1) (layer "F.Cu") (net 2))
 (segment (start 165.1 96.52) (end 165.1 114.3) (width 1) (layer "F.Cu") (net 2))
 (segment (start 144.78 127) (end 139.7 132.08) (width 1) (layer "F.Cu") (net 2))
 (segment (start 162.1 123.16) (end 158.26 127) (width 1) (layer "F.Cu") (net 2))
 (segment (start 170.18 114.3) (end 165.1 114.3) (width 1) (layer "F.Cu") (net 2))
 (segment (start 144.78 121.92) (end 144.78 127) (width 1) (layer "F.Cu") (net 2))
 (segment (start 162.56 114.3) (end 152.4 114.3) (width 1) (layer "F.Cu") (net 2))
 (segment (start 139.7 132.08) (end 134.62 132.08) (width 1) (layer "F.Cu") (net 2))
 (segment (start 149.86 127) (end 144.78 127) (width 1) (layer "F.Cu") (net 2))
 (segment (start 165.1 76.2) (end 165.1 93.98) (width 1) (layer "F.Cu") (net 2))
 (segment (start 114.3 76.2) (end 104.14 76.2) (width 1) (layer "F.Cu") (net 2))
 (segment (start 165.1 101.6) (end 165.1 93.98) (width 1) (layer "F.Cu") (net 2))
 (segment (start 114.3 132.08) (end 104.14 132.08) (width 1) (layer "F.Cu") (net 2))
 (segment (start 152.4 114.3) (end 144.78 121.92) (width 1) (layer "F.Cu") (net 2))
 (segment (start 170.18 114.3) (end 175.26 114.3) (width 1) (layer "F.Cu") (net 2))
 (segment (start 182.88 101.6) (end 182.88 86.36) (width 1) (layer "F.Cu") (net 1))
 (segment (start 114.3 81.28) (end 104.14 81.28) (width 1) (layer "F.Cu") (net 35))
 (segment (start 114.3 86.36) (end 104.14 86.36) (width 1) (layer "F.Cu") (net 37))
 (segment (start 114.3 96.52) (end 104.14 96.52) (width 1) (layer "F.Cu") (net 41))
 (segment (start 114.3 99.06) (end 104.14 99.06) (width 1) (layer "F.Cu") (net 42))
 (segment (start 114.3 106.68) (end 104.14 106.68) (width 1) (layer "F.Cu") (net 45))
 (segment (start 114.3 83.82) (end 104.14 83.82) (width 1) (layer "F.Cu") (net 36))
 (segment (start 114.3 101.6) (end 104.14 101.6) (width 1) (layer "F.Cu") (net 43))
 (segment (start 114.3 93.98) (end 104.14 93.98) (width 1) (layer "F.Cu") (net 40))
 (segment (start 114.3 104.14) (end 104.14 104.14) (width 1) (layer "F.Cu") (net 44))
 (segment (start 114.3 78.74) (end 104.14 78.74) (width 1) (layer "F.Cu") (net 34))
 (segment (start 114.3 88.9) (end 104.14 88.9) (width 1) (layer "F.Cu") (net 38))
 (segment (start 114.3 91.44) (end 104.14 91.44) (width 1) (layer "F.Cu") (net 39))
 (segment (start 121.92 114.3) (end 121.92 127.16) (width 1) (layer "F.Cu") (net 5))
 (segment (start 124.3 129.54) (end 134.62 129.54) (width 1) (layer "F.Cu") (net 5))
 (segment (start 149.86 73.66) (end 139.7 73.66) (width 1) (layer "F.Cu") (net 5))
 (segment (start 162.56 76.2) (end 162.56 93.98) (width 1) (layer "F.Cu") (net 5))
 (segment (start 162.56 101.6) (end 162.56 93.98) (width 1) (layer "F.Cu") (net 5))
 (segment (start 134.62 101.6) (end 121.92 114.3) (width 1) (layer "F.Cu") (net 5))
 (segment (start 162.56 76.2) (end 152.4 76.2) (width 1) (layer "F.Cu") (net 5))
 (segment (start 134.62 78.74) (end 134.62 101.6) (width 1) (layer "F.Cu") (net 5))
 (segment (start 152.4 76.2) (end 149.86 73.66) (width 1) (layer "F.Cu") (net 5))
 (segment (start 121.92 127.16) (end 124.3 129.54) (width 1) (layer "F.Cu") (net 5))
 (segment (start 139.7 73.66) (end 134.62 78.74) (width 1) (layer "F.Cu") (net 5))
 (segment (start 139.7 86.36) (end 149.86 86.36) (width 1) (layer "F.Cu") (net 16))
 (segment (start 149.86 104.14) (end 139.7 104.14) (width 1) (layer "F.Cu") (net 23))
 (segment (start 139.7 96.52) (end 149.86 96.52) (width 1) (layer "F.Cu") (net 20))
 (segment (start 139.7 101.6) (end 149.86 101.6) (width 1) (layer "F.Cu") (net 22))
 (segment (start 149.86 88.9) (end 139.7 88.9) (width 1) (layer "F.Cu") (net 17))
 (segment (start 149.86 93.98) (end 139.7 93.98) (width 1) (layer "F.Cu") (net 19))
 (segment (start 149.86 99.06) (end 139.7 99.06) (width 1) (layer "F.Cu") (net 21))
 (segment (start 139.7 91.44) (end 149.86 91.44) (width 1) (layer "F.Cu") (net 18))
 (segment (start 149.86 78.74) (end 139.7 78.74) (width 1) (layer "F.Cu") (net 13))
 (segment (start 139.7 83.82) (end 149.86 83.82) (width 1) (layer "F.Cu") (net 15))
 (segment (start 139.7 106.68) (end 149.86 106.68) (width 1) (layer "F.Cu") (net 24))
 (segment (start 139.7 81.28) (end 149.86 81.28) (width 1) (layer "F.Cu") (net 14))
 (segment (start 164.18 132.08) (end 149.86 132.08) (width 1) (layer "F.Cu") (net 28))
 (segment (start 165.1 131.16) (end 164.18 132.08) (width 1) (layer "F.Cu") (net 28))
 (segment (start 165.1 128.62) (end 150.78 128.62) (width 1) (layer "F.Cu") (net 27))
 (segment (start 150.78 128.62) (end 149.86 129.54) (width 1) (layer "F.Cu") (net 27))
 (segment (start 165.1 137.16) (end 149.86 137.16) (width 1) (layer "F.Cu") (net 30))
 (segment (start 165.1 134.62) (end 149.86 134.62) (width 1) (layer "F.Cu") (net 29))
 (segment (start 189.58 128.62) (end 190.5 129.54) (width 0.2) (layer "F.Cu") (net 47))
 (segment (start 178.9 128.62) (end 189.58 128.62) (width 1) (layer "F.Cu") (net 47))
 (segment (start 178.9 131.16) (end 179.82 132.08) (width 0.2) (layer "F.Cu") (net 48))
 (segment (start 179.82 132.08) (end 190.5 132.08) (width 1) (layer "F.Cu") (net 48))
 (segment (start 178.9 134.62) (end 190.5 134.62) (width 1) (layer "F.Cu") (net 31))
 (segment (start 178.9 137.16) (end 190.5 137.16) (width 1) (layer "F.Cu") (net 32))
 (segment (start 104.14 137.16) (end 114.3 137.16) (width 1) (layer "F.Cu") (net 12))
 (segment (start 114.3 124.46) (end 104.14 124.46) (width 1) (layer "F.Cu") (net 8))
 (segment (start 104.14 134.62) (end 114.3 134.62) (width 1) (layer "F.Cu") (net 11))
 (segment (start 104.14 127) (end 114.3 127) (width 1) (layer "F.Cu") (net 9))
 (segment (start 124.3 124.46) (end 134.62 124.46) (width 1) (layer "F.Cu") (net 3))
 (segment (start 124.3 137.16) (end 134.62 137.16) (width 1) (layer "F.Cu") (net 7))
 (segment (start 124.3 134.62) (end 134.62 134.62) (width 1) (layer "F.Cu") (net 6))
 (segment (start 124.3 127) (end 134.62 127) (width 1) (layer "F.Cu") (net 4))
 (segment (start 119.38 124.46) (end 114.3 129.54) (width 1) (layer "F.Cu") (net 10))
 (segment (start 114.3 73.66) (end 119.38 78.74) (width 1) (layer "F.Cu") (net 10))
 (segment (start 104.14 129.54) (end 114.3 129.54) (width 1) (layer "F.Cu") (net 10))
 (segment (start 114.3 73.66) (end 104.14 73.66) (width 1) (layer "F.Cu") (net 10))
 (segment (start 119.38 78.74) (end 119.38 124.46) (width 1) (layer "F.Cu") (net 10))
 (segment (start 139.7 109.22) (end 149.86 109.22) (width 1) (layer "F.Cu") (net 25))
 (segment (start 114.3 109.22) (end 104.14 109.22) (width 1) (layer "F.Cu") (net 46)))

